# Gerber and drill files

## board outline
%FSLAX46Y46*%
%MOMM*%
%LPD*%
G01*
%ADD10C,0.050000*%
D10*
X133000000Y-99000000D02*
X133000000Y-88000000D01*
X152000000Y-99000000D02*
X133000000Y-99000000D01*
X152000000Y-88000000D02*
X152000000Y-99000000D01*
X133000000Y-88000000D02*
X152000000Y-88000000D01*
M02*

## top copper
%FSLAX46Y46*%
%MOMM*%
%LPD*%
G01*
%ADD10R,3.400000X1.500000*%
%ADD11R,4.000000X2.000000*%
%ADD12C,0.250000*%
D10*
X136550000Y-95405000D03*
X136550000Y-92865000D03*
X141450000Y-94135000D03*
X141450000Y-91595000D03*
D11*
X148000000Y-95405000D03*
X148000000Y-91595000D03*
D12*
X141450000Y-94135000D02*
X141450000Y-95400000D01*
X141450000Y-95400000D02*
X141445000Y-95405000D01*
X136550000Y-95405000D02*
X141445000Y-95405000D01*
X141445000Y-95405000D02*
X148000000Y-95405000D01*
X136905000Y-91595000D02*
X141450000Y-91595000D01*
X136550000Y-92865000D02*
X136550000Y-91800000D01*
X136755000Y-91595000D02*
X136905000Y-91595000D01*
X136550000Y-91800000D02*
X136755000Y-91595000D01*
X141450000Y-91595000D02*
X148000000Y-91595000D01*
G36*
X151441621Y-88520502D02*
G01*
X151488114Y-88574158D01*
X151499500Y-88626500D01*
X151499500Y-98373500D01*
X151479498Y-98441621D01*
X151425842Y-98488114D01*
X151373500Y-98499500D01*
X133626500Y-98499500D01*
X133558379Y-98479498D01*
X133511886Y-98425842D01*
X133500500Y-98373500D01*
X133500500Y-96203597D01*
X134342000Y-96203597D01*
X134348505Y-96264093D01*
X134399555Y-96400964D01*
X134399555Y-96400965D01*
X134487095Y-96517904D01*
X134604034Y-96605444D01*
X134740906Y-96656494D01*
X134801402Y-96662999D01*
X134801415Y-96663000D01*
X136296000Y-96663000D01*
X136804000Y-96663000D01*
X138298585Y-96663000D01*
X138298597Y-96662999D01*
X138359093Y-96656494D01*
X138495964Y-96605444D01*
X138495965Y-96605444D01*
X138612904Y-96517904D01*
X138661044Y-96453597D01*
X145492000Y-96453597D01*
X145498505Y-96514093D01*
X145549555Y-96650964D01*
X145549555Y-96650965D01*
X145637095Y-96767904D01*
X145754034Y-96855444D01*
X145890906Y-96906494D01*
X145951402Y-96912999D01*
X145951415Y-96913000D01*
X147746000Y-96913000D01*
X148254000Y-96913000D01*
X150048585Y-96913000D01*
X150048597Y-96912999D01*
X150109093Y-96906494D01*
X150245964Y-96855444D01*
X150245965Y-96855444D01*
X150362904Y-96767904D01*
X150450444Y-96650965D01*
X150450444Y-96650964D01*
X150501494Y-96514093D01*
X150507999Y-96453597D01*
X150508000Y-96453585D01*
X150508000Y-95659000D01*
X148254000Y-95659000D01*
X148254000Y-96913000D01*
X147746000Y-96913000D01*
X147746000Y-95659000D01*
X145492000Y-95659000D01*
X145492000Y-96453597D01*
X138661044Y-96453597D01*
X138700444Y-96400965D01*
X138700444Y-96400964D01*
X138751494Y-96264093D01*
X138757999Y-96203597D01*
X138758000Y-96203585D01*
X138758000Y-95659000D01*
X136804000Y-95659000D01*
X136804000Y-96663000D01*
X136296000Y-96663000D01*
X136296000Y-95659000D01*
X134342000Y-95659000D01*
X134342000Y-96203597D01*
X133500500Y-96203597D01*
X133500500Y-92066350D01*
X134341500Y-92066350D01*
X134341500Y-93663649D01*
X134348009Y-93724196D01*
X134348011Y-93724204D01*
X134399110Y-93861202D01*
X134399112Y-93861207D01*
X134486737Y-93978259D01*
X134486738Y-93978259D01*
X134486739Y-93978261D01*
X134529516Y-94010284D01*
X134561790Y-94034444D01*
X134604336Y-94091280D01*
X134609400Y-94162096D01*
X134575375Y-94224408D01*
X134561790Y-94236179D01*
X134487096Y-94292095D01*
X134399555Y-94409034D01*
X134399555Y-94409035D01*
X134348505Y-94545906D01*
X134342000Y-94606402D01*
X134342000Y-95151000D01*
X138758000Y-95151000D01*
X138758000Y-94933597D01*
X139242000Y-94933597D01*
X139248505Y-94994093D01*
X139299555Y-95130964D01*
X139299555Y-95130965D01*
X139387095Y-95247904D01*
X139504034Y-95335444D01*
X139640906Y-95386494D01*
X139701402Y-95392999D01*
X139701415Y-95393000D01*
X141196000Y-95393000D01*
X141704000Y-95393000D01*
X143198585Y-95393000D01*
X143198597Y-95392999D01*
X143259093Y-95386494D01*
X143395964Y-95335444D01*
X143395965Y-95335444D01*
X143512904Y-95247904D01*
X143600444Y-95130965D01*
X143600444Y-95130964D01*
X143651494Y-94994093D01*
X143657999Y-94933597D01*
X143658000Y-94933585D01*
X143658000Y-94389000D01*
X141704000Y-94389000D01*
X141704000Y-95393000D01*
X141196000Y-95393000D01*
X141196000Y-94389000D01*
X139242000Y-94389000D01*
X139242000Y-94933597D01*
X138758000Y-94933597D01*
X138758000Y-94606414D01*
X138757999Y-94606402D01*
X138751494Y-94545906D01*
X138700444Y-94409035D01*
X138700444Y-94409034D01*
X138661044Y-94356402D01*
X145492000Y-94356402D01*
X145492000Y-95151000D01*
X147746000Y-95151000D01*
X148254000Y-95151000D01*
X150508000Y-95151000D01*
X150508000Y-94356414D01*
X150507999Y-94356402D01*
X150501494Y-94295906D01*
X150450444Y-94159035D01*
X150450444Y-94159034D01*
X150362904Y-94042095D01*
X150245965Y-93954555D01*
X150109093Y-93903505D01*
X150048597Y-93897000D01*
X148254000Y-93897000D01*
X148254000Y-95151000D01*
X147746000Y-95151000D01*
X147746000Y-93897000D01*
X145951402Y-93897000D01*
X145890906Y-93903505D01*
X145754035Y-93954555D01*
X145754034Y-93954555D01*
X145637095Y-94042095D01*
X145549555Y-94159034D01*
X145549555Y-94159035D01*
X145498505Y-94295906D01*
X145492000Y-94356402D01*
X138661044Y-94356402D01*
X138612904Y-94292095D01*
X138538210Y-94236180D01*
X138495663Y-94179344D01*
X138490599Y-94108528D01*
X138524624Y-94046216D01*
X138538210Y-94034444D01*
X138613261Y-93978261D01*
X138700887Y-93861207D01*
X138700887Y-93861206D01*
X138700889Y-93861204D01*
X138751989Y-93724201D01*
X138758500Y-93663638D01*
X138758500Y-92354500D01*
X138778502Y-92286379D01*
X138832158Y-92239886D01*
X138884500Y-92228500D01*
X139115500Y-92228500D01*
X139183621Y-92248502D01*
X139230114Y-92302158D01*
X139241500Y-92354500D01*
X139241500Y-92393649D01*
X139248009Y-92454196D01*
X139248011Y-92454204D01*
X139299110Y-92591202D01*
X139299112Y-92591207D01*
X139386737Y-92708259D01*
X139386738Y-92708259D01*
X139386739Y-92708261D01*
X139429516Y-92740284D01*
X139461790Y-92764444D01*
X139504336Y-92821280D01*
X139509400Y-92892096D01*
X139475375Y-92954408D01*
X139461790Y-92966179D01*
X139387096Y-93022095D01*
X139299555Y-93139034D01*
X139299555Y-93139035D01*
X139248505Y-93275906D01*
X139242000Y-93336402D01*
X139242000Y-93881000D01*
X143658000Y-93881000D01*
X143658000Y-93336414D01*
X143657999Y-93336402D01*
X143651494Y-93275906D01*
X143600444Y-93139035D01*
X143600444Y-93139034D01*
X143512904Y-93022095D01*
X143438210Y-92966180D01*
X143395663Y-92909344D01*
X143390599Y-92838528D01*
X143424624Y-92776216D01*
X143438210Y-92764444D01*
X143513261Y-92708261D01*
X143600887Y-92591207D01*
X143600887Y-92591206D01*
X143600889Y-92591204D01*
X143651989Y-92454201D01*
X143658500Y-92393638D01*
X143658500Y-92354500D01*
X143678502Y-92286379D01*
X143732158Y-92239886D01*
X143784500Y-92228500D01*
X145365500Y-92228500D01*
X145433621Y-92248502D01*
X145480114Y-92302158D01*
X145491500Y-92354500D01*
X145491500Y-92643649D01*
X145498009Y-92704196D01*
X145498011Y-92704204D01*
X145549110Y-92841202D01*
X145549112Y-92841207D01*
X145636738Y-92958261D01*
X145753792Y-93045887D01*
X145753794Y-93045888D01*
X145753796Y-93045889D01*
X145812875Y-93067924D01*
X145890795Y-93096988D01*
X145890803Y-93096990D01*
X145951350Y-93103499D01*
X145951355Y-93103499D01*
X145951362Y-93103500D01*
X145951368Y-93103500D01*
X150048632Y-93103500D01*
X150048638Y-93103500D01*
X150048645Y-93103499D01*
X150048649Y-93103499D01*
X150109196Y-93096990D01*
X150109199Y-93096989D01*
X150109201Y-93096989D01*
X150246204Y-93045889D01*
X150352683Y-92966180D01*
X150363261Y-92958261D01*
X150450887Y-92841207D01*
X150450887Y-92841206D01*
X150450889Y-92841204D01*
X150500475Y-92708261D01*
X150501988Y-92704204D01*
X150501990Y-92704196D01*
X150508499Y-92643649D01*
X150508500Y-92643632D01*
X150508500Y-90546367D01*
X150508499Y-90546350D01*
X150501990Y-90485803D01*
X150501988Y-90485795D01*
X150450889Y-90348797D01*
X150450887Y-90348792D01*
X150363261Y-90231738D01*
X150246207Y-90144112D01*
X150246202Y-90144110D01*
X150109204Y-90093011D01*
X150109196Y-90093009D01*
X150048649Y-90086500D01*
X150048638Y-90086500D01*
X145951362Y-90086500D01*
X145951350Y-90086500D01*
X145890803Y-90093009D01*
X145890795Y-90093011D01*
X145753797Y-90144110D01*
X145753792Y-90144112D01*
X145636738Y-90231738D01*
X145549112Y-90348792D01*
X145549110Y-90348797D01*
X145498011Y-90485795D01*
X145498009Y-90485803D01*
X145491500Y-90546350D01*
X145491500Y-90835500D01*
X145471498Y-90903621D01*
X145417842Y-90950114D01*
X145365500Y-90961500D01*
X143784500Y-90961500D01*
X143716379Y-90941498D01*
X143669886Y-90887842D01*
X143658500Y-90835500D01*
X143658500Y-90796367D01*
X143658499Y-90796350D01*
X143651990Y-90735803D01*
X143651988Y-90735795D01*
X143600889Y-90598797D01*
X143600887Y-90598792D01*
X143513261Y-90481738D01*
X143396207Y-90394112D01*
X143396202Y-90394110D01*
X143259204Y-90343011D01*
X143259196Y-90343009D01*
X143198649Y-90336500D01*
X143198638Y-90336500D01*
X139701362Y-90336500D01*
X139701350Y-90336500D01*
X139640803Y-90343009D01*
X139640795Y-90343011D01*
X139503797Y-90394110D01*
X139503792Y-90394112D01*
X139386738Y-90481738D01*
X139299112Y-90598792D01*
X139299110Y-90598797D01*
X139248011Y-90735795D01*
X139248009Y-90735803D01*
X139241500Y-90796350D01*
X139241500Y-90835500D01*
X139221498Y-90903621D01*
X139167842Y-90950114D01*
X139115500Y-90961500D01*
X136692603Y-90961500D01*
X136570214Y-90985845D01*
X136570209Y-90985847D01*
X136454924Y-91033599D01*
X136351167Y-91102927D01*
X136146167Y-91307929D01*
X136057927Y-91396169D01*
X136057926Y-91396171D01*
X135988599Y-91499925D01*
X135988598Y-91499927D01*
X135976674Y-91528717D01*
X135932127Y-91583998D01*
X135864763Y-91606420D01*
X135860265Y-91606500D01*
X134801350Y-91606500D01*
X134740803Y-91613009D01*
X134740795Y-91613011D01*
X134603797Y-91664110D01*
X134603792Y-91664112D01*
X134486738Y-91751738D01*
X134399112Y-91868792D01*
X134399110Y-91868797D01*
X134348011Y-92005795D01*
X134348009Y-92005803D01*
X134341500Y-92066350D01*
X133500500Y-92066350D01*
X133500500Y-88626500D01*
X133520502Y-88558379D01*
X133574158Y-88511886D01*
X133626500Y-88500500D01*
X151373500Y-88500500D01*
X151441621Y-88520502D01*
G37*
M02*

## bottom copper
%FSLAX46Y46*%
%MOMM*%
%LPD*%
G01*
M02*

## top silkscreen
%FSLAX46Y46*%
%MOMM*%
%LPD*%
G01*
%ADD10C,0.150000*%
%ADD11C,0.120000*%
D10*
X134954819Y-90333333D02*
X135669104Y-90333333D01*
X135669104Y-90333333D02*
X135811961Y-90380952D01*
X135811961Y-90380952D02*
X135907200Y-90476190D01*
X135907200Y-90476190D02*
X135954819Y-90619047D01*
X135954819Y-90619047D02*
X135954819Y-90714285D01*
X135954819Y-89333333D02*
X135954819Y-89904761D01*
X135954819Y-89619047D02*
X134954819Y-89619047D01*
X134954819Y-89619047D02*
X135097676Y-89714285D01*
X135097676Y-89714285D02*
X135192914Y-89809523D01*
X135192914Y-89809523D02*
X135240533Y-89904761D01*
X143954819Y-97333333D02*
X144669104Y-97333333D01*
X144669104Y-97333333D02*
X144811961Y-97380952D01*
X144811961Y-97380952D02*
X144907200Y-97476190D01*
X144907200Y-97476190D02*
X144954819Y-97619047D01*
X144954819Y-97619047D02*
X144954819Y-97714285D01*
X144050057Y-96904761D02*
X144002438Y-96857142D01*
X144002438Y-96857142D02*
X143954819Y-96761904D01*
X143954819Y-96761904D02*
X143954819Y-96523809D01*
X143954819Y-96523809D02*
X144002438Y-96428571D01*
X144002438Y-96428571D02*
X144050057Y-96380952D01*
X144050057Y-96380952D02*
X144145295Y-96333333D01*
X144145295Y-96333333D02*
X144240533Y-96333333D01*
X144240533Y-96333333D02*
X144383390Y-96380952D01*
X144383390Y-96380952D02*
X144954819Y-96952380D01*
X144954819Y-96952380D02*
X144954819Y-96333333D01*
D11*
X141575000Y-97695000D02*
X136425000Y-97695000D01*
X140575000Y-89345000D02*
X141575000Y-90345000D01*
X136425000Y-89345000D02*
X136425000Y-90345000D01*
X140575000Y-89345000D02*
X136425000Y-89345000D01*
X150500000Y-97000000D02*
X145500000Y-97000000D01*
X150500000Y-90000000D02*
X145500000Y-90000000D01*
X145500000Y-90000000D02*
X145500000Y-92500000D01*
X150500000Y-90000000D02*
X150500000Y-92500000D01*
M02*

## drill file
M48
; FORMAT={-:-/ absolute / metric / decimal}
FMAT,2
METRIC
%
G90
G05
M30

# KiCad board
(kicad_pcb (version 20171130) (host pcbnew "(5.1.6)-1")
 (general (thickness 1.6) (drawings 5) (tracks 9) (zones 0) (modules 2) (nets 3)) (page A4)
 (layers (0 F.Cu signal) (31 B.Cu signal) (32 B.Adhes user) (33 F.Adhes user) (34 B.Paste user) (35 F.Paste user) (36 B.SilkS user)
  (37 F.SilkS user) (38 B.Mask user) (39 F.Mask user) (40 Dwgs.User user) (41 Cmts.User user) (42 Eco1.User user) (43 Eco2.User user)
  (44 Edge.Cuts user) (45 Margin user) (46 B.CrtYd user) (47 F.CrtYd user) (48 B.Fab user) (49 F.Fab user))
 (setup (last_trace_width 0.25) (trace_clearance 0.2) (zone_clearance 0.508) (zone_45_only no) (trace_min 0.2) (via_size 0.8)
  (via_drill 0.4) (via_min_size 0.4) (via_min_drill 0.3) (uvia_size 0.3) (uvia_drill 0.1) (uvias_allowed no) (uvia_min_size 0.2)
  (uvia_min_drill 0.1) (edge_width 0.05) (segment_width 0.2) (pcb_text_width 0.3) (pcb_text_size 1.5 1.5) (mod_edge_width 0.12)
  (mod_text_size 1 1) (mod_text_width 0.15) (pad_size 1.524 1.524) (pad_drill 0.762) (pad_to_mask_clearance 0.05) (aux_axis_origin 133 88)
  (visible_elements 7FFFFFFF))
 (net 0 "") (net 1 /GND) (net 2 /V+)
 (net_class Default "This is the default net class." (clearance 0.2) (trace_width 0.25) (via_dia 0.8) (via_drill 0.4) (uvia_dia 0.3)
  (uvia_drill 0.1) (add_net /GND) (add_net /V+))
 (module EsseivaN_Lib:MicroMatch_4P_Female (layer F.Cu) (at 139 93.5 270)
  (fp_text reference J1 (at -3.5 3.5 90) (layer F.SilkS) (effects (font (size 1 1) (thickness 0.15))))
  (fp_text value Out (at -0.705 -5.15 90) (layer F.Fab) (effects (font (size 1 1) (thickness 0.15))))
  (fp_line (start 4.195 -2.575) (end 4.195 2.575) (layer F.SilkS) (width 0.12))
  (fp_line (start -4.155 -1.575) (end -3.155 -2.575) (layer F.SilkS) (width 0.12))
  (fp_line (start -4.155 2.575) (end -3.155 2.575) (layer F.SilkS) (width 0.12))
  (fp_line (start -4.155 -1.575) (end -4.155 2.575) (layer F.SilkS) (width 0.12))
  (pad 4 smd rect (at 1.905 2.45 90) (size 1.5 3.4) (layers F.Cu F.Paste F.Mask) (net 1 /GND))
  (pad 2 smd rect (at -0.635 2.45 90) (size 1.5 3.4) (layers F.Cu F.Paste F.Mask) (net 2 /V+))
  (pad 3 smd rect (at 0.635 -2.45 90) (size 1.5 3.4) (layers F.Cu F.Paste F.Mask) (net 1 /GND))
  (pad 1 smd rect (at -1.905 -2.45 90) (size 1.5 3.4) (layers F.Cu F.Paste F.Mask) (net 2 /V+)))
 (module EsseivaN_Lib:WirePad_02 (layer F.Cu) (at 148 93.5 270)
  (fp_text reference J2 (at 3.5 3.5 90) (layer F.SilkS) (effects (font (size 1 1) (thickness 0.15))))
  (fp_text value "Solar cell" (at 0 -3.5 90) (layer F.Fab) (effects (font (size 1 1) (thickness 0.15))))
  (fp_line (start 3.5 -2.5) (end 3.5 2.5) (layer F.SilkS) (width 0.12))
  (fp_line (start -3.5 -2.5) (end -3.5 2.5) (layer F.SilkS) (width 0.12))
  (fp_line (start -3.5 2.5) (end -1 2.5) (layer F.SilkS) (width 0.12))
  (fp_line (start -3.5 -2.5) (end -1 -2.5) (layer F.SilkS) (width 0.12))
  (pad 2 connect rect (at 1.905 0 270) (size 2 4) (layers F.Cu F.Mask) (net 1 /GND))
  (pad 1 connect rect (at -1.905 0 270) (size 2 4) (layers F.Cu F.Mask) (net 2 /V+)))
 (gr_line (start 133 99) (end 133 88) (layer Edge.Cuts) (width 0.05))
 (gr_line (start 152 99) (end 133 99) (layer Edge.Cuts) (width 0.05))
 (gr_line (start 152 88) (end 152 99) (layer Edge.Cuts) (width 0.05))
 (gr_line (start 133 88) (end 152 88) (layer Edge.Cuts) (width 0.05))
 (segment (start 141.45 94.135) (end 141.45 95.4) (width 0.25) (layer F.Cu) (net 1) (status 10))
 (segment (start 141.45 95.4) (end 141.445 95.405) (width 0.25) (layer F.Cu) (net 1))
 (segment (start 136.55 95.405) (end 141.445 95.405) (width 0.25) (layer F.Cu) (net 1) (status 10))
 (segment (start 141.445 95.405) (end 148 95.405) (width 0.25) (layer F.Cu) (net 1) (status 20))
 (segment (start 136.905 91.595) (end 141.45 91.595) (width 0.25) (layer F.Cu) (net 2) (status 20))
 (segment (start 136.55 92.865) (end 136.55 91.8) (width 0.25) (layer F.Cu) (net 2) (status 10))
 (segment (start 136.755 91.595) (end 136.905 91.595) (width 0.25) (layer F.Cu) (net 2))
 (segment (start 136.55 91.8) (end 136.755 91.595) (width 0.25) (layer F.Cu) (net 2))
 (segment (start 141.45 91.595) (end 148 91.595) (width 0.25) (layer F.Cu) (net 2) (status 30))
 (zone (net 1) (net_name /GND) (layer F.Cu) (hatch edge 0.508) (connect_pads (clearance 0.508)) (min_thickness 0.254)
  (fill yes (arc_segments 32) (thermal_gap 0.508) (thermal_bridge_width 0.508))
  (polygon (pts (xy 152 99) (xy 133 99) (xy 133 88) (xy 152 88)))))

